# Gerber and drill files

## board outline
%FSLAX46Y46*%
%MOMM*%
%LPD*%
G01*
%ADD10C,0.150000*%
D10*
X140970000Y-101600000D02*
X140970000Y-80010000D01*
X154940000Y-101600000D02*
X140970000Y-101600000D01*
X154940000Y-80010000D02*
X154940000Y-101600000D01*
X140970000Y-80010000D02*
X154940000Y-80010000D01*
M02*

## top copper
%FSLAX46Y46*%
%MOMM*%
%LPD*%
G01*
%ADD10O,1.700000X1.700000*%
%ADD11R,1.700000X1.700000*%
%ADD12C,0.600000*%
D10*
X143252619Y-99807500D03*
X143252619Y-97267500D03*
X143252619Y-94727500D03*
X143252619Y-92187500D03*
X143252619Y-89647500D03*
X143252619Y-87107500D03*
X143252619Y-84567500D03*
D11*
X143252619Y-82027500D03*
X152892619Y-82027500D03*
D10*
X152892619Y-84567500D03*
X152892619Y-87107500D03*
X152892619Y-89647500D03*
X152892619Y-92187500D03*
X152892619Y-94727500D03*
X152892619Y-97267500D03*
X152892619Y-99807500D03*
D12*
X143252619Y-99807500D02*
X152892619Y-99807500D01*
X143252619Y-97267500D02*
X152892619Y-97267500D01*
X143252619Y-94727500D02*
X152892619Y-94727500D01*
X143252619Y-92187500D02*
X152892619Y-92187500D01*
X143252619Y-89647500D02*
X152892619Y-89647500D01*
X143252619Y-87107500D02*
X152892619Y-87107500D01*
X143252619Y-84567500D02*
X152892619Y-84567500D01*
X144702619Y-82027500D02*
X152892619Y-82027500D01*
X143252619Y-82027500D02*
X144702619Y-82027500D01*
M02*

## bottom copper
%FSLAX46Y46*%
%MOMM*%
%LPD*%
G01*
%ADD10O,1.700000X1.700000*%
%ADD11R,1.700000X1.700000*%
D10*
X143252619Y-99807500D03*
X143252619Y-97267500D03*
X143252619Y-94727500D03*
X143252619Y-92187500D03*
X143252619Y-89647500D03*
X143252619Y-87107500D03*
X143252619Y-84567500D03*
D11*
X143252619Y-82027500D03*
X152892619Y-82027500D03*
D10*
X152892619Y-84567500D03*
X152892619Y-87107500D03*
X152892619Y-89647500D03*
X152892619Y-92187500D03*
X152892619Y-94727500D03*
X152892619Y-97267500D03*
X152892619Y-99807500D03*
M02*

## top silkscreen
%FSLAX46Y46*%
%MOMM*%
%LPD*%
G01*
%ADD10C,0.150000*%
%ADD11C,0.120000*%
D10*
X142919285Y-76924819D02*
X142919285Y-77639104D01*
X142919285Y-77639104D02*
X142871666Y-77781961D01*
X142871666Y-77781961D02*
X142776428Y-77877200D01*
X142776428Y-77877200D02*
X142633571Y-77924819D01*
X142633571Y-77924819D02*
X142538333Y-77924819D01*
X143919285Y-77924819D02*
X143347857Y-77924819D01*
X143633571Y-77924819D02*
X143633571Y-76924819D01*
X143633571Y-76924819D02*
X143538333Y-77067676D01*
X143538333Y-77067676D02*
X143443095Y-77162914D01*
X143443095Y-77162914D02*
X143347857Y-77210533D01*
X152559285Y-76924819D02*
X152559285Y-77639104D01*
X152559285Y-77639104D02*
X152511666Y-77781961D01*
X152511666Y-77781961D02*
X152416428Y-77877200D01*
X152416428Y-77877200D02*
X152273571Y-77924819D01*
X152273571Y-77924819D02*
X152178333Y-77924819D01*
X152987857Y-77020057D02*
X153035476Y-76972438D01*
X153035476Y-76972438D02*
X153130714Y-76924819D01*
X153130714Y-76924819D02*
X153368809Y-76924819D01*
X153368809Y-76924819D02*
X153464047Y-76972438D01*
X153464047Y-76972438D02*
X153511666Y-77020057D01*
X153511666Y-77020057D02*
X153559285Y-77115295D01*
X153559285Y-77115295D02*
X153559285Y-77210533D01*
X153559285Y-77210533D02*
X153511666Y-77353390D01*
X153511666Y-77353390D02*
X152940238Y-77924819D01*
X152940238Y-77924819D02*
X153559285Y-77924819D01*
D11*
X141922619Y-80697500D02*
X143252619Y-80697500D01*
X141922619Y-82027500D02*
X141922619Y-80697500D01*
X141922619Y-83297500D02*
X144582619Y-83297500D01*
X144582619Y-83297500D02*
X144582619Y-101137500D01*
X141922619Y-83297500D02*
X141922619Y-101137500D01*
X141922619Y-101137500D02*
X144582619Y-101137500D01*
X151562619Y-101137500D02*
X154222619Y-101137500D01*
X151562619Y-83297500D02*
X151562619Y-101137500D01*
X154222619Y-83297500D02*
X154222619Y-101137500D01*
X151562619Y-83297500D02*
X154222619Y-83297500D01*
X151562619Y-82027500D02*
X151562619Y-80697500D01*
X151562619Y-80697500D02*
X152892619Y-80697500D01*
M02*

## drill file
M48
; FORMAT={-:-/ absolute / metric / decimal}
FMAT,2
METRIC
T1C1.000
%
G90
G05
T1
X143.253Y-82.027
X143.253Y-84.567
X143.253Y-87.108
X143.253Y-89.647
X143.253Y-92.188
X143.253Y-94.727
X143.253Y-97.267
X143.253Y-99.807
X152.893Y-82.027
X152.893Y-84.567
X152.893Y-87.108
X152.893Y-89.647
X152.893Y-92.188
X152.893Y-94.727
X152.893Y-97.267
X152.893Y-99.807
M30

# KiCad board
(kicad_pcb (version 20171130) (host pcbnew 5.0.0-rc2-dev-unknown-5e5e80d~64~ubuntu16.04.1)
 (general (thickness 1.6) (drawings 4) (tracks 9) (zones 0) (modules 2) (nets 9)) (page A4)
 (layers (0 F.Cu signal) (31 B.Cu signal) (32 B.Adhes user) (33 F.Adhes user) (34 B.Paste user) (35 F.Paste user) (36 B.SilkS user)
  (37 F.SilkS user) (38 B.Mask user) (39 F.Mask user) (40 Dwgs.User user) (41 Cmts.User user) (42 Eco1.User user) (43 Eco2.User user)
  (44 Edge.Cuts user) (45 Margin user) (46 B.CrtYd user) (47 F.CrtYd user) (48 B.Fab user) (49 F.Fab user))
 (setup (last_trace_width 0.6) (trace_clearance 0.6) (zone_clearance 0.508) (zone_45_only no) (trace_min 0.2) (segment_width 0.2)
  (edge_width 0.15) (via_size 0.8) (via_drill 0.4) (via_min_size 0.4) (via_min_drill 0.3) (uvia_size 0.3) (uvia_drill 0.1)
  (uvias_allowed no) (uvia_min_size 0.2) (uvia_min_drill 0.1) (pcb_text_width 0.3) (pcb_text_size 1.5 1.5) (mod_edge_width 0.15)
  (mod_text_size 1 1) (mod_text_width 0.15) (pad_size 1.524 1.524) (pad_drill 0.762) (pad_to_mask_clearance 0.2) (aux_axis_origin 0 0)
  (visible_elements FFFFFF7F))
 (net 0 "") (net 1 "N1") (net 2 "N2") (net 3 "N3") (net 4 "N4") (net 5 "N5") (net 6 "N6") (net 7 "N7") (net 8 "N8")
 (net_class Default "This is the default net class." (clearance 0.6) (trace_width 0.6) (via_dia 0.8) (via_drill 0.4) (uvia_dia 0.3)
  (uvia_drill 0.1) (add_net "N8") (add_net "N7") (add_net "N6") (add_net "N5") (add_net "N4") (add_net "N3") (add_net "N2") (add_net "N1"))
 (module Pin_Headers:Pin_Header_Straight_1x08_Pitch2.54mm (layer F.Cu) (at 143.252619 82.0275)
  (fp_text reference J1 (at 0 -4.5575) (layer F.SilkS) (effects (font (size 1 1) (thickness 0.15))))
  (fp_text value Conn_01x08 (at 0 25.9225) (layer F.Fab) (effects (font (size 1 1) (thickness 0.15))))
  (fp_line (start -1.33 -1.33) (end 0 -1.33) (layer F.SilkS) (width 0.12))
  (fp_line (start -1.33 0) (end -1.33 -1.33) (layer F.SilkS) (width 0.12))
  (fp_line (start -1.33 1.27) (end 1.33 1.27) (layer F.SilkS) (width 0.12))
  (fp_line (start 1.33 1.27) (end 1.33 19.11) (layer F.SilkS) (width 0.12))
  (fp_line (start -1.33 1.27) (end -1.33 19.11) (layer F.SilkS) (width 0.12))
  (fp_line (start -1.33 19.11) (end 1.33 19.11) (layer F.SilkS) (width 0.12))
  (pad 8 thru_hole oval (at 0 17.78) (size 1.7 1.7) (drill 1) (layers *.Cu *.Mask) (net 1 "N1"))
  (pad 7 thru_hole oval (at 0 15.24) (size 1.7 1.7) (drill 1) (layers *.Cu *.Mask) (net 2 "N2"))
  (pad 6 thru_hole oval (at 0 12.7) (size 1.7 1.7) (drill 1) (layers *.Cu *.Mask) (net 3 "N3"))
  (pad 5 thru_hole oval (at 0 10.16) (size 1.7 1.7) (drill 1) (layers *.Cu *.Mask) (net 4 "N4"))
  (pad 4 thru_hole oval (at 0 7.62) (size 1.7 1.7) (drill 1) (layers *.Cu *.Mask) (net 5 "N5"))
  (pad 3 thru_hole oval (at 0 5.08) (size 1.7 1.7) (drill 1) (layers *.Cu *.Mask) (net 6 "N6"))
  (pad 2 thru_hole oval (at 0 2.54) (size 1.7 1.7) (drill 1) (layers *.Cu *.Mask) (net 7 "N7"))
  (pad 1 thru_hole rect (at 0 0) (size 1.7 1.7) (drill 1) (layers *.Cu *.Mask) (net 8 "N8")))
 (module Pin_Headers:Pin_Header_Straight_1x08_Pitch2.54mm (layer F.Cu) (at 152.892619 82.0275)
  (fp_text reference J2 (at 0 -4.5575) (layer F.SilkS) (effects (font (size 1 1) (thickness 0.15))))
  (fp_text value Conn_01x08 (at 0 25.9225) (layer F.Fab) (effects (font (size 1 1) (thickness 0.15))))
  (fp_line (start -1.33 19.11) (end 1.33 19.11) (layer F.SilkS) (width 0.12))
  (fp_line (start -1.33 1.27) (end -1.33 19.11) (layer F.SilkS) (width 0.12))
  (fp_line (start 1.33 1.27) (end 1.33 19.11) (layer F.SilkS) (width 0.12))
  (fp_line (start -1.33 1.27) (end 1.33 1.27) (layer F.SilkS) (width 0.12))
  (fp_line (start -1.33 0) (end -1.33 -1.33) (layer F.SilkS) (width 0.12))
  (fp_line (start -1.33 -1.33) (end 0 -1.33) (layer F.SilkS) (width 0.12))
  (pad 1 thru_hole rect (at 0 0) (size 1.7 1.7) (drill 1) (layers *.Cu *.Mask) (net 8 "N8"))
  (pad 2 thru_hole oval (at 0 2.54) (size 1.7 1.7) (drill 1) (layers *.Cu *.Mask) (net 7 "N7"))
  (pad 3 thru_hole oval (at 0 5.08) (size 1.7 1.7) (drill 1) (layers *.Cu *.Mask) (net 6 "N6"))
  (pad 4 thru_hole oval (at 0 7.62) (size 1.7 1.7) (drill 1) (layers *.Cu *.Mask) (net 5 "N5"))
  (pad 5 thru_hole oval (at 0 10.16) (size 1.7 1.7) (drill 1) (layers *.Cu *.Mask) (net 4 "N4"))
  (pad 6 thru_hole oval (at 0 12.7) (size 1.7 1.7) (drill 1) (layers *.Cu *.Mask) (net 3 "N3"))
  (pad 7 thru_hole oval (at 0 15.24) (size 1.7 1.7) (drill 1) (layers *.Cu *.Mask) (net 2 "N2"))
  (pad 8 thru_hole oval (at 0 17.78) (size 1.7 1.7) (drill 1) (layers *.Cu *.Mask) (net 1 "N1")))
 (gr_line (start 140.97 101.6) (end 140.97 80.01) (layer Edge.Cuts) (width 0.15))
 (gr_line (start 154.94 101.6) (end 140.97 101.6) (layer Edge.Cuts) (width 0.15))
 (gr_line (start 154.94 80.01) (end 154.94 101.6) (layer Edge.Cuts) (width 0.15))
 (gr_line (start 140.97 80.01) (end 154.94 80.01) (layer Edge.Cuts) (width 0.15))
 (segment (start 143.252619 99.8075) (end 152.892619 99.8075) (width 0.6) (layer F.Cu) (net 1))
 (segment (start 143.252619 97.2675) (end 152.892619 97.2675) (width 0.6) (layer F.Cu) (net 2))
 (segment (start 143.252619 94.7275) (end 152.892619 94.7275) (width 0.6) (layer F.Cu) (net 3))
 (segment (start 143.252619 92.1875) (end 152.892619 92.1875) (width 0.6) (layer F.Cu) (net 4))
 (segment (start 143.252619 89.6475) (end 152.892619 89.6475) (width 0.6) (layer F.Cu) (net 5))
 (segment (start 143.252619 87.1075) (end 152.892619 87.1075) (width 0.6) (layer F.Cu) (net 6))
 (segment (start 143.252619 84.5675) (end 152.892619 84.5675) (width 0.6) (layer F.Cu) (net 7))
 (segment (start 144.702619 82.0275) (end 152.892619 82.0275) (width 0.6) (layer F.Cu) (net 8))
 (segment (start 143.252619 82.0275) (end 144.702619 82.0275) (width 0.6) (layer F.Cu) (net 8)))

